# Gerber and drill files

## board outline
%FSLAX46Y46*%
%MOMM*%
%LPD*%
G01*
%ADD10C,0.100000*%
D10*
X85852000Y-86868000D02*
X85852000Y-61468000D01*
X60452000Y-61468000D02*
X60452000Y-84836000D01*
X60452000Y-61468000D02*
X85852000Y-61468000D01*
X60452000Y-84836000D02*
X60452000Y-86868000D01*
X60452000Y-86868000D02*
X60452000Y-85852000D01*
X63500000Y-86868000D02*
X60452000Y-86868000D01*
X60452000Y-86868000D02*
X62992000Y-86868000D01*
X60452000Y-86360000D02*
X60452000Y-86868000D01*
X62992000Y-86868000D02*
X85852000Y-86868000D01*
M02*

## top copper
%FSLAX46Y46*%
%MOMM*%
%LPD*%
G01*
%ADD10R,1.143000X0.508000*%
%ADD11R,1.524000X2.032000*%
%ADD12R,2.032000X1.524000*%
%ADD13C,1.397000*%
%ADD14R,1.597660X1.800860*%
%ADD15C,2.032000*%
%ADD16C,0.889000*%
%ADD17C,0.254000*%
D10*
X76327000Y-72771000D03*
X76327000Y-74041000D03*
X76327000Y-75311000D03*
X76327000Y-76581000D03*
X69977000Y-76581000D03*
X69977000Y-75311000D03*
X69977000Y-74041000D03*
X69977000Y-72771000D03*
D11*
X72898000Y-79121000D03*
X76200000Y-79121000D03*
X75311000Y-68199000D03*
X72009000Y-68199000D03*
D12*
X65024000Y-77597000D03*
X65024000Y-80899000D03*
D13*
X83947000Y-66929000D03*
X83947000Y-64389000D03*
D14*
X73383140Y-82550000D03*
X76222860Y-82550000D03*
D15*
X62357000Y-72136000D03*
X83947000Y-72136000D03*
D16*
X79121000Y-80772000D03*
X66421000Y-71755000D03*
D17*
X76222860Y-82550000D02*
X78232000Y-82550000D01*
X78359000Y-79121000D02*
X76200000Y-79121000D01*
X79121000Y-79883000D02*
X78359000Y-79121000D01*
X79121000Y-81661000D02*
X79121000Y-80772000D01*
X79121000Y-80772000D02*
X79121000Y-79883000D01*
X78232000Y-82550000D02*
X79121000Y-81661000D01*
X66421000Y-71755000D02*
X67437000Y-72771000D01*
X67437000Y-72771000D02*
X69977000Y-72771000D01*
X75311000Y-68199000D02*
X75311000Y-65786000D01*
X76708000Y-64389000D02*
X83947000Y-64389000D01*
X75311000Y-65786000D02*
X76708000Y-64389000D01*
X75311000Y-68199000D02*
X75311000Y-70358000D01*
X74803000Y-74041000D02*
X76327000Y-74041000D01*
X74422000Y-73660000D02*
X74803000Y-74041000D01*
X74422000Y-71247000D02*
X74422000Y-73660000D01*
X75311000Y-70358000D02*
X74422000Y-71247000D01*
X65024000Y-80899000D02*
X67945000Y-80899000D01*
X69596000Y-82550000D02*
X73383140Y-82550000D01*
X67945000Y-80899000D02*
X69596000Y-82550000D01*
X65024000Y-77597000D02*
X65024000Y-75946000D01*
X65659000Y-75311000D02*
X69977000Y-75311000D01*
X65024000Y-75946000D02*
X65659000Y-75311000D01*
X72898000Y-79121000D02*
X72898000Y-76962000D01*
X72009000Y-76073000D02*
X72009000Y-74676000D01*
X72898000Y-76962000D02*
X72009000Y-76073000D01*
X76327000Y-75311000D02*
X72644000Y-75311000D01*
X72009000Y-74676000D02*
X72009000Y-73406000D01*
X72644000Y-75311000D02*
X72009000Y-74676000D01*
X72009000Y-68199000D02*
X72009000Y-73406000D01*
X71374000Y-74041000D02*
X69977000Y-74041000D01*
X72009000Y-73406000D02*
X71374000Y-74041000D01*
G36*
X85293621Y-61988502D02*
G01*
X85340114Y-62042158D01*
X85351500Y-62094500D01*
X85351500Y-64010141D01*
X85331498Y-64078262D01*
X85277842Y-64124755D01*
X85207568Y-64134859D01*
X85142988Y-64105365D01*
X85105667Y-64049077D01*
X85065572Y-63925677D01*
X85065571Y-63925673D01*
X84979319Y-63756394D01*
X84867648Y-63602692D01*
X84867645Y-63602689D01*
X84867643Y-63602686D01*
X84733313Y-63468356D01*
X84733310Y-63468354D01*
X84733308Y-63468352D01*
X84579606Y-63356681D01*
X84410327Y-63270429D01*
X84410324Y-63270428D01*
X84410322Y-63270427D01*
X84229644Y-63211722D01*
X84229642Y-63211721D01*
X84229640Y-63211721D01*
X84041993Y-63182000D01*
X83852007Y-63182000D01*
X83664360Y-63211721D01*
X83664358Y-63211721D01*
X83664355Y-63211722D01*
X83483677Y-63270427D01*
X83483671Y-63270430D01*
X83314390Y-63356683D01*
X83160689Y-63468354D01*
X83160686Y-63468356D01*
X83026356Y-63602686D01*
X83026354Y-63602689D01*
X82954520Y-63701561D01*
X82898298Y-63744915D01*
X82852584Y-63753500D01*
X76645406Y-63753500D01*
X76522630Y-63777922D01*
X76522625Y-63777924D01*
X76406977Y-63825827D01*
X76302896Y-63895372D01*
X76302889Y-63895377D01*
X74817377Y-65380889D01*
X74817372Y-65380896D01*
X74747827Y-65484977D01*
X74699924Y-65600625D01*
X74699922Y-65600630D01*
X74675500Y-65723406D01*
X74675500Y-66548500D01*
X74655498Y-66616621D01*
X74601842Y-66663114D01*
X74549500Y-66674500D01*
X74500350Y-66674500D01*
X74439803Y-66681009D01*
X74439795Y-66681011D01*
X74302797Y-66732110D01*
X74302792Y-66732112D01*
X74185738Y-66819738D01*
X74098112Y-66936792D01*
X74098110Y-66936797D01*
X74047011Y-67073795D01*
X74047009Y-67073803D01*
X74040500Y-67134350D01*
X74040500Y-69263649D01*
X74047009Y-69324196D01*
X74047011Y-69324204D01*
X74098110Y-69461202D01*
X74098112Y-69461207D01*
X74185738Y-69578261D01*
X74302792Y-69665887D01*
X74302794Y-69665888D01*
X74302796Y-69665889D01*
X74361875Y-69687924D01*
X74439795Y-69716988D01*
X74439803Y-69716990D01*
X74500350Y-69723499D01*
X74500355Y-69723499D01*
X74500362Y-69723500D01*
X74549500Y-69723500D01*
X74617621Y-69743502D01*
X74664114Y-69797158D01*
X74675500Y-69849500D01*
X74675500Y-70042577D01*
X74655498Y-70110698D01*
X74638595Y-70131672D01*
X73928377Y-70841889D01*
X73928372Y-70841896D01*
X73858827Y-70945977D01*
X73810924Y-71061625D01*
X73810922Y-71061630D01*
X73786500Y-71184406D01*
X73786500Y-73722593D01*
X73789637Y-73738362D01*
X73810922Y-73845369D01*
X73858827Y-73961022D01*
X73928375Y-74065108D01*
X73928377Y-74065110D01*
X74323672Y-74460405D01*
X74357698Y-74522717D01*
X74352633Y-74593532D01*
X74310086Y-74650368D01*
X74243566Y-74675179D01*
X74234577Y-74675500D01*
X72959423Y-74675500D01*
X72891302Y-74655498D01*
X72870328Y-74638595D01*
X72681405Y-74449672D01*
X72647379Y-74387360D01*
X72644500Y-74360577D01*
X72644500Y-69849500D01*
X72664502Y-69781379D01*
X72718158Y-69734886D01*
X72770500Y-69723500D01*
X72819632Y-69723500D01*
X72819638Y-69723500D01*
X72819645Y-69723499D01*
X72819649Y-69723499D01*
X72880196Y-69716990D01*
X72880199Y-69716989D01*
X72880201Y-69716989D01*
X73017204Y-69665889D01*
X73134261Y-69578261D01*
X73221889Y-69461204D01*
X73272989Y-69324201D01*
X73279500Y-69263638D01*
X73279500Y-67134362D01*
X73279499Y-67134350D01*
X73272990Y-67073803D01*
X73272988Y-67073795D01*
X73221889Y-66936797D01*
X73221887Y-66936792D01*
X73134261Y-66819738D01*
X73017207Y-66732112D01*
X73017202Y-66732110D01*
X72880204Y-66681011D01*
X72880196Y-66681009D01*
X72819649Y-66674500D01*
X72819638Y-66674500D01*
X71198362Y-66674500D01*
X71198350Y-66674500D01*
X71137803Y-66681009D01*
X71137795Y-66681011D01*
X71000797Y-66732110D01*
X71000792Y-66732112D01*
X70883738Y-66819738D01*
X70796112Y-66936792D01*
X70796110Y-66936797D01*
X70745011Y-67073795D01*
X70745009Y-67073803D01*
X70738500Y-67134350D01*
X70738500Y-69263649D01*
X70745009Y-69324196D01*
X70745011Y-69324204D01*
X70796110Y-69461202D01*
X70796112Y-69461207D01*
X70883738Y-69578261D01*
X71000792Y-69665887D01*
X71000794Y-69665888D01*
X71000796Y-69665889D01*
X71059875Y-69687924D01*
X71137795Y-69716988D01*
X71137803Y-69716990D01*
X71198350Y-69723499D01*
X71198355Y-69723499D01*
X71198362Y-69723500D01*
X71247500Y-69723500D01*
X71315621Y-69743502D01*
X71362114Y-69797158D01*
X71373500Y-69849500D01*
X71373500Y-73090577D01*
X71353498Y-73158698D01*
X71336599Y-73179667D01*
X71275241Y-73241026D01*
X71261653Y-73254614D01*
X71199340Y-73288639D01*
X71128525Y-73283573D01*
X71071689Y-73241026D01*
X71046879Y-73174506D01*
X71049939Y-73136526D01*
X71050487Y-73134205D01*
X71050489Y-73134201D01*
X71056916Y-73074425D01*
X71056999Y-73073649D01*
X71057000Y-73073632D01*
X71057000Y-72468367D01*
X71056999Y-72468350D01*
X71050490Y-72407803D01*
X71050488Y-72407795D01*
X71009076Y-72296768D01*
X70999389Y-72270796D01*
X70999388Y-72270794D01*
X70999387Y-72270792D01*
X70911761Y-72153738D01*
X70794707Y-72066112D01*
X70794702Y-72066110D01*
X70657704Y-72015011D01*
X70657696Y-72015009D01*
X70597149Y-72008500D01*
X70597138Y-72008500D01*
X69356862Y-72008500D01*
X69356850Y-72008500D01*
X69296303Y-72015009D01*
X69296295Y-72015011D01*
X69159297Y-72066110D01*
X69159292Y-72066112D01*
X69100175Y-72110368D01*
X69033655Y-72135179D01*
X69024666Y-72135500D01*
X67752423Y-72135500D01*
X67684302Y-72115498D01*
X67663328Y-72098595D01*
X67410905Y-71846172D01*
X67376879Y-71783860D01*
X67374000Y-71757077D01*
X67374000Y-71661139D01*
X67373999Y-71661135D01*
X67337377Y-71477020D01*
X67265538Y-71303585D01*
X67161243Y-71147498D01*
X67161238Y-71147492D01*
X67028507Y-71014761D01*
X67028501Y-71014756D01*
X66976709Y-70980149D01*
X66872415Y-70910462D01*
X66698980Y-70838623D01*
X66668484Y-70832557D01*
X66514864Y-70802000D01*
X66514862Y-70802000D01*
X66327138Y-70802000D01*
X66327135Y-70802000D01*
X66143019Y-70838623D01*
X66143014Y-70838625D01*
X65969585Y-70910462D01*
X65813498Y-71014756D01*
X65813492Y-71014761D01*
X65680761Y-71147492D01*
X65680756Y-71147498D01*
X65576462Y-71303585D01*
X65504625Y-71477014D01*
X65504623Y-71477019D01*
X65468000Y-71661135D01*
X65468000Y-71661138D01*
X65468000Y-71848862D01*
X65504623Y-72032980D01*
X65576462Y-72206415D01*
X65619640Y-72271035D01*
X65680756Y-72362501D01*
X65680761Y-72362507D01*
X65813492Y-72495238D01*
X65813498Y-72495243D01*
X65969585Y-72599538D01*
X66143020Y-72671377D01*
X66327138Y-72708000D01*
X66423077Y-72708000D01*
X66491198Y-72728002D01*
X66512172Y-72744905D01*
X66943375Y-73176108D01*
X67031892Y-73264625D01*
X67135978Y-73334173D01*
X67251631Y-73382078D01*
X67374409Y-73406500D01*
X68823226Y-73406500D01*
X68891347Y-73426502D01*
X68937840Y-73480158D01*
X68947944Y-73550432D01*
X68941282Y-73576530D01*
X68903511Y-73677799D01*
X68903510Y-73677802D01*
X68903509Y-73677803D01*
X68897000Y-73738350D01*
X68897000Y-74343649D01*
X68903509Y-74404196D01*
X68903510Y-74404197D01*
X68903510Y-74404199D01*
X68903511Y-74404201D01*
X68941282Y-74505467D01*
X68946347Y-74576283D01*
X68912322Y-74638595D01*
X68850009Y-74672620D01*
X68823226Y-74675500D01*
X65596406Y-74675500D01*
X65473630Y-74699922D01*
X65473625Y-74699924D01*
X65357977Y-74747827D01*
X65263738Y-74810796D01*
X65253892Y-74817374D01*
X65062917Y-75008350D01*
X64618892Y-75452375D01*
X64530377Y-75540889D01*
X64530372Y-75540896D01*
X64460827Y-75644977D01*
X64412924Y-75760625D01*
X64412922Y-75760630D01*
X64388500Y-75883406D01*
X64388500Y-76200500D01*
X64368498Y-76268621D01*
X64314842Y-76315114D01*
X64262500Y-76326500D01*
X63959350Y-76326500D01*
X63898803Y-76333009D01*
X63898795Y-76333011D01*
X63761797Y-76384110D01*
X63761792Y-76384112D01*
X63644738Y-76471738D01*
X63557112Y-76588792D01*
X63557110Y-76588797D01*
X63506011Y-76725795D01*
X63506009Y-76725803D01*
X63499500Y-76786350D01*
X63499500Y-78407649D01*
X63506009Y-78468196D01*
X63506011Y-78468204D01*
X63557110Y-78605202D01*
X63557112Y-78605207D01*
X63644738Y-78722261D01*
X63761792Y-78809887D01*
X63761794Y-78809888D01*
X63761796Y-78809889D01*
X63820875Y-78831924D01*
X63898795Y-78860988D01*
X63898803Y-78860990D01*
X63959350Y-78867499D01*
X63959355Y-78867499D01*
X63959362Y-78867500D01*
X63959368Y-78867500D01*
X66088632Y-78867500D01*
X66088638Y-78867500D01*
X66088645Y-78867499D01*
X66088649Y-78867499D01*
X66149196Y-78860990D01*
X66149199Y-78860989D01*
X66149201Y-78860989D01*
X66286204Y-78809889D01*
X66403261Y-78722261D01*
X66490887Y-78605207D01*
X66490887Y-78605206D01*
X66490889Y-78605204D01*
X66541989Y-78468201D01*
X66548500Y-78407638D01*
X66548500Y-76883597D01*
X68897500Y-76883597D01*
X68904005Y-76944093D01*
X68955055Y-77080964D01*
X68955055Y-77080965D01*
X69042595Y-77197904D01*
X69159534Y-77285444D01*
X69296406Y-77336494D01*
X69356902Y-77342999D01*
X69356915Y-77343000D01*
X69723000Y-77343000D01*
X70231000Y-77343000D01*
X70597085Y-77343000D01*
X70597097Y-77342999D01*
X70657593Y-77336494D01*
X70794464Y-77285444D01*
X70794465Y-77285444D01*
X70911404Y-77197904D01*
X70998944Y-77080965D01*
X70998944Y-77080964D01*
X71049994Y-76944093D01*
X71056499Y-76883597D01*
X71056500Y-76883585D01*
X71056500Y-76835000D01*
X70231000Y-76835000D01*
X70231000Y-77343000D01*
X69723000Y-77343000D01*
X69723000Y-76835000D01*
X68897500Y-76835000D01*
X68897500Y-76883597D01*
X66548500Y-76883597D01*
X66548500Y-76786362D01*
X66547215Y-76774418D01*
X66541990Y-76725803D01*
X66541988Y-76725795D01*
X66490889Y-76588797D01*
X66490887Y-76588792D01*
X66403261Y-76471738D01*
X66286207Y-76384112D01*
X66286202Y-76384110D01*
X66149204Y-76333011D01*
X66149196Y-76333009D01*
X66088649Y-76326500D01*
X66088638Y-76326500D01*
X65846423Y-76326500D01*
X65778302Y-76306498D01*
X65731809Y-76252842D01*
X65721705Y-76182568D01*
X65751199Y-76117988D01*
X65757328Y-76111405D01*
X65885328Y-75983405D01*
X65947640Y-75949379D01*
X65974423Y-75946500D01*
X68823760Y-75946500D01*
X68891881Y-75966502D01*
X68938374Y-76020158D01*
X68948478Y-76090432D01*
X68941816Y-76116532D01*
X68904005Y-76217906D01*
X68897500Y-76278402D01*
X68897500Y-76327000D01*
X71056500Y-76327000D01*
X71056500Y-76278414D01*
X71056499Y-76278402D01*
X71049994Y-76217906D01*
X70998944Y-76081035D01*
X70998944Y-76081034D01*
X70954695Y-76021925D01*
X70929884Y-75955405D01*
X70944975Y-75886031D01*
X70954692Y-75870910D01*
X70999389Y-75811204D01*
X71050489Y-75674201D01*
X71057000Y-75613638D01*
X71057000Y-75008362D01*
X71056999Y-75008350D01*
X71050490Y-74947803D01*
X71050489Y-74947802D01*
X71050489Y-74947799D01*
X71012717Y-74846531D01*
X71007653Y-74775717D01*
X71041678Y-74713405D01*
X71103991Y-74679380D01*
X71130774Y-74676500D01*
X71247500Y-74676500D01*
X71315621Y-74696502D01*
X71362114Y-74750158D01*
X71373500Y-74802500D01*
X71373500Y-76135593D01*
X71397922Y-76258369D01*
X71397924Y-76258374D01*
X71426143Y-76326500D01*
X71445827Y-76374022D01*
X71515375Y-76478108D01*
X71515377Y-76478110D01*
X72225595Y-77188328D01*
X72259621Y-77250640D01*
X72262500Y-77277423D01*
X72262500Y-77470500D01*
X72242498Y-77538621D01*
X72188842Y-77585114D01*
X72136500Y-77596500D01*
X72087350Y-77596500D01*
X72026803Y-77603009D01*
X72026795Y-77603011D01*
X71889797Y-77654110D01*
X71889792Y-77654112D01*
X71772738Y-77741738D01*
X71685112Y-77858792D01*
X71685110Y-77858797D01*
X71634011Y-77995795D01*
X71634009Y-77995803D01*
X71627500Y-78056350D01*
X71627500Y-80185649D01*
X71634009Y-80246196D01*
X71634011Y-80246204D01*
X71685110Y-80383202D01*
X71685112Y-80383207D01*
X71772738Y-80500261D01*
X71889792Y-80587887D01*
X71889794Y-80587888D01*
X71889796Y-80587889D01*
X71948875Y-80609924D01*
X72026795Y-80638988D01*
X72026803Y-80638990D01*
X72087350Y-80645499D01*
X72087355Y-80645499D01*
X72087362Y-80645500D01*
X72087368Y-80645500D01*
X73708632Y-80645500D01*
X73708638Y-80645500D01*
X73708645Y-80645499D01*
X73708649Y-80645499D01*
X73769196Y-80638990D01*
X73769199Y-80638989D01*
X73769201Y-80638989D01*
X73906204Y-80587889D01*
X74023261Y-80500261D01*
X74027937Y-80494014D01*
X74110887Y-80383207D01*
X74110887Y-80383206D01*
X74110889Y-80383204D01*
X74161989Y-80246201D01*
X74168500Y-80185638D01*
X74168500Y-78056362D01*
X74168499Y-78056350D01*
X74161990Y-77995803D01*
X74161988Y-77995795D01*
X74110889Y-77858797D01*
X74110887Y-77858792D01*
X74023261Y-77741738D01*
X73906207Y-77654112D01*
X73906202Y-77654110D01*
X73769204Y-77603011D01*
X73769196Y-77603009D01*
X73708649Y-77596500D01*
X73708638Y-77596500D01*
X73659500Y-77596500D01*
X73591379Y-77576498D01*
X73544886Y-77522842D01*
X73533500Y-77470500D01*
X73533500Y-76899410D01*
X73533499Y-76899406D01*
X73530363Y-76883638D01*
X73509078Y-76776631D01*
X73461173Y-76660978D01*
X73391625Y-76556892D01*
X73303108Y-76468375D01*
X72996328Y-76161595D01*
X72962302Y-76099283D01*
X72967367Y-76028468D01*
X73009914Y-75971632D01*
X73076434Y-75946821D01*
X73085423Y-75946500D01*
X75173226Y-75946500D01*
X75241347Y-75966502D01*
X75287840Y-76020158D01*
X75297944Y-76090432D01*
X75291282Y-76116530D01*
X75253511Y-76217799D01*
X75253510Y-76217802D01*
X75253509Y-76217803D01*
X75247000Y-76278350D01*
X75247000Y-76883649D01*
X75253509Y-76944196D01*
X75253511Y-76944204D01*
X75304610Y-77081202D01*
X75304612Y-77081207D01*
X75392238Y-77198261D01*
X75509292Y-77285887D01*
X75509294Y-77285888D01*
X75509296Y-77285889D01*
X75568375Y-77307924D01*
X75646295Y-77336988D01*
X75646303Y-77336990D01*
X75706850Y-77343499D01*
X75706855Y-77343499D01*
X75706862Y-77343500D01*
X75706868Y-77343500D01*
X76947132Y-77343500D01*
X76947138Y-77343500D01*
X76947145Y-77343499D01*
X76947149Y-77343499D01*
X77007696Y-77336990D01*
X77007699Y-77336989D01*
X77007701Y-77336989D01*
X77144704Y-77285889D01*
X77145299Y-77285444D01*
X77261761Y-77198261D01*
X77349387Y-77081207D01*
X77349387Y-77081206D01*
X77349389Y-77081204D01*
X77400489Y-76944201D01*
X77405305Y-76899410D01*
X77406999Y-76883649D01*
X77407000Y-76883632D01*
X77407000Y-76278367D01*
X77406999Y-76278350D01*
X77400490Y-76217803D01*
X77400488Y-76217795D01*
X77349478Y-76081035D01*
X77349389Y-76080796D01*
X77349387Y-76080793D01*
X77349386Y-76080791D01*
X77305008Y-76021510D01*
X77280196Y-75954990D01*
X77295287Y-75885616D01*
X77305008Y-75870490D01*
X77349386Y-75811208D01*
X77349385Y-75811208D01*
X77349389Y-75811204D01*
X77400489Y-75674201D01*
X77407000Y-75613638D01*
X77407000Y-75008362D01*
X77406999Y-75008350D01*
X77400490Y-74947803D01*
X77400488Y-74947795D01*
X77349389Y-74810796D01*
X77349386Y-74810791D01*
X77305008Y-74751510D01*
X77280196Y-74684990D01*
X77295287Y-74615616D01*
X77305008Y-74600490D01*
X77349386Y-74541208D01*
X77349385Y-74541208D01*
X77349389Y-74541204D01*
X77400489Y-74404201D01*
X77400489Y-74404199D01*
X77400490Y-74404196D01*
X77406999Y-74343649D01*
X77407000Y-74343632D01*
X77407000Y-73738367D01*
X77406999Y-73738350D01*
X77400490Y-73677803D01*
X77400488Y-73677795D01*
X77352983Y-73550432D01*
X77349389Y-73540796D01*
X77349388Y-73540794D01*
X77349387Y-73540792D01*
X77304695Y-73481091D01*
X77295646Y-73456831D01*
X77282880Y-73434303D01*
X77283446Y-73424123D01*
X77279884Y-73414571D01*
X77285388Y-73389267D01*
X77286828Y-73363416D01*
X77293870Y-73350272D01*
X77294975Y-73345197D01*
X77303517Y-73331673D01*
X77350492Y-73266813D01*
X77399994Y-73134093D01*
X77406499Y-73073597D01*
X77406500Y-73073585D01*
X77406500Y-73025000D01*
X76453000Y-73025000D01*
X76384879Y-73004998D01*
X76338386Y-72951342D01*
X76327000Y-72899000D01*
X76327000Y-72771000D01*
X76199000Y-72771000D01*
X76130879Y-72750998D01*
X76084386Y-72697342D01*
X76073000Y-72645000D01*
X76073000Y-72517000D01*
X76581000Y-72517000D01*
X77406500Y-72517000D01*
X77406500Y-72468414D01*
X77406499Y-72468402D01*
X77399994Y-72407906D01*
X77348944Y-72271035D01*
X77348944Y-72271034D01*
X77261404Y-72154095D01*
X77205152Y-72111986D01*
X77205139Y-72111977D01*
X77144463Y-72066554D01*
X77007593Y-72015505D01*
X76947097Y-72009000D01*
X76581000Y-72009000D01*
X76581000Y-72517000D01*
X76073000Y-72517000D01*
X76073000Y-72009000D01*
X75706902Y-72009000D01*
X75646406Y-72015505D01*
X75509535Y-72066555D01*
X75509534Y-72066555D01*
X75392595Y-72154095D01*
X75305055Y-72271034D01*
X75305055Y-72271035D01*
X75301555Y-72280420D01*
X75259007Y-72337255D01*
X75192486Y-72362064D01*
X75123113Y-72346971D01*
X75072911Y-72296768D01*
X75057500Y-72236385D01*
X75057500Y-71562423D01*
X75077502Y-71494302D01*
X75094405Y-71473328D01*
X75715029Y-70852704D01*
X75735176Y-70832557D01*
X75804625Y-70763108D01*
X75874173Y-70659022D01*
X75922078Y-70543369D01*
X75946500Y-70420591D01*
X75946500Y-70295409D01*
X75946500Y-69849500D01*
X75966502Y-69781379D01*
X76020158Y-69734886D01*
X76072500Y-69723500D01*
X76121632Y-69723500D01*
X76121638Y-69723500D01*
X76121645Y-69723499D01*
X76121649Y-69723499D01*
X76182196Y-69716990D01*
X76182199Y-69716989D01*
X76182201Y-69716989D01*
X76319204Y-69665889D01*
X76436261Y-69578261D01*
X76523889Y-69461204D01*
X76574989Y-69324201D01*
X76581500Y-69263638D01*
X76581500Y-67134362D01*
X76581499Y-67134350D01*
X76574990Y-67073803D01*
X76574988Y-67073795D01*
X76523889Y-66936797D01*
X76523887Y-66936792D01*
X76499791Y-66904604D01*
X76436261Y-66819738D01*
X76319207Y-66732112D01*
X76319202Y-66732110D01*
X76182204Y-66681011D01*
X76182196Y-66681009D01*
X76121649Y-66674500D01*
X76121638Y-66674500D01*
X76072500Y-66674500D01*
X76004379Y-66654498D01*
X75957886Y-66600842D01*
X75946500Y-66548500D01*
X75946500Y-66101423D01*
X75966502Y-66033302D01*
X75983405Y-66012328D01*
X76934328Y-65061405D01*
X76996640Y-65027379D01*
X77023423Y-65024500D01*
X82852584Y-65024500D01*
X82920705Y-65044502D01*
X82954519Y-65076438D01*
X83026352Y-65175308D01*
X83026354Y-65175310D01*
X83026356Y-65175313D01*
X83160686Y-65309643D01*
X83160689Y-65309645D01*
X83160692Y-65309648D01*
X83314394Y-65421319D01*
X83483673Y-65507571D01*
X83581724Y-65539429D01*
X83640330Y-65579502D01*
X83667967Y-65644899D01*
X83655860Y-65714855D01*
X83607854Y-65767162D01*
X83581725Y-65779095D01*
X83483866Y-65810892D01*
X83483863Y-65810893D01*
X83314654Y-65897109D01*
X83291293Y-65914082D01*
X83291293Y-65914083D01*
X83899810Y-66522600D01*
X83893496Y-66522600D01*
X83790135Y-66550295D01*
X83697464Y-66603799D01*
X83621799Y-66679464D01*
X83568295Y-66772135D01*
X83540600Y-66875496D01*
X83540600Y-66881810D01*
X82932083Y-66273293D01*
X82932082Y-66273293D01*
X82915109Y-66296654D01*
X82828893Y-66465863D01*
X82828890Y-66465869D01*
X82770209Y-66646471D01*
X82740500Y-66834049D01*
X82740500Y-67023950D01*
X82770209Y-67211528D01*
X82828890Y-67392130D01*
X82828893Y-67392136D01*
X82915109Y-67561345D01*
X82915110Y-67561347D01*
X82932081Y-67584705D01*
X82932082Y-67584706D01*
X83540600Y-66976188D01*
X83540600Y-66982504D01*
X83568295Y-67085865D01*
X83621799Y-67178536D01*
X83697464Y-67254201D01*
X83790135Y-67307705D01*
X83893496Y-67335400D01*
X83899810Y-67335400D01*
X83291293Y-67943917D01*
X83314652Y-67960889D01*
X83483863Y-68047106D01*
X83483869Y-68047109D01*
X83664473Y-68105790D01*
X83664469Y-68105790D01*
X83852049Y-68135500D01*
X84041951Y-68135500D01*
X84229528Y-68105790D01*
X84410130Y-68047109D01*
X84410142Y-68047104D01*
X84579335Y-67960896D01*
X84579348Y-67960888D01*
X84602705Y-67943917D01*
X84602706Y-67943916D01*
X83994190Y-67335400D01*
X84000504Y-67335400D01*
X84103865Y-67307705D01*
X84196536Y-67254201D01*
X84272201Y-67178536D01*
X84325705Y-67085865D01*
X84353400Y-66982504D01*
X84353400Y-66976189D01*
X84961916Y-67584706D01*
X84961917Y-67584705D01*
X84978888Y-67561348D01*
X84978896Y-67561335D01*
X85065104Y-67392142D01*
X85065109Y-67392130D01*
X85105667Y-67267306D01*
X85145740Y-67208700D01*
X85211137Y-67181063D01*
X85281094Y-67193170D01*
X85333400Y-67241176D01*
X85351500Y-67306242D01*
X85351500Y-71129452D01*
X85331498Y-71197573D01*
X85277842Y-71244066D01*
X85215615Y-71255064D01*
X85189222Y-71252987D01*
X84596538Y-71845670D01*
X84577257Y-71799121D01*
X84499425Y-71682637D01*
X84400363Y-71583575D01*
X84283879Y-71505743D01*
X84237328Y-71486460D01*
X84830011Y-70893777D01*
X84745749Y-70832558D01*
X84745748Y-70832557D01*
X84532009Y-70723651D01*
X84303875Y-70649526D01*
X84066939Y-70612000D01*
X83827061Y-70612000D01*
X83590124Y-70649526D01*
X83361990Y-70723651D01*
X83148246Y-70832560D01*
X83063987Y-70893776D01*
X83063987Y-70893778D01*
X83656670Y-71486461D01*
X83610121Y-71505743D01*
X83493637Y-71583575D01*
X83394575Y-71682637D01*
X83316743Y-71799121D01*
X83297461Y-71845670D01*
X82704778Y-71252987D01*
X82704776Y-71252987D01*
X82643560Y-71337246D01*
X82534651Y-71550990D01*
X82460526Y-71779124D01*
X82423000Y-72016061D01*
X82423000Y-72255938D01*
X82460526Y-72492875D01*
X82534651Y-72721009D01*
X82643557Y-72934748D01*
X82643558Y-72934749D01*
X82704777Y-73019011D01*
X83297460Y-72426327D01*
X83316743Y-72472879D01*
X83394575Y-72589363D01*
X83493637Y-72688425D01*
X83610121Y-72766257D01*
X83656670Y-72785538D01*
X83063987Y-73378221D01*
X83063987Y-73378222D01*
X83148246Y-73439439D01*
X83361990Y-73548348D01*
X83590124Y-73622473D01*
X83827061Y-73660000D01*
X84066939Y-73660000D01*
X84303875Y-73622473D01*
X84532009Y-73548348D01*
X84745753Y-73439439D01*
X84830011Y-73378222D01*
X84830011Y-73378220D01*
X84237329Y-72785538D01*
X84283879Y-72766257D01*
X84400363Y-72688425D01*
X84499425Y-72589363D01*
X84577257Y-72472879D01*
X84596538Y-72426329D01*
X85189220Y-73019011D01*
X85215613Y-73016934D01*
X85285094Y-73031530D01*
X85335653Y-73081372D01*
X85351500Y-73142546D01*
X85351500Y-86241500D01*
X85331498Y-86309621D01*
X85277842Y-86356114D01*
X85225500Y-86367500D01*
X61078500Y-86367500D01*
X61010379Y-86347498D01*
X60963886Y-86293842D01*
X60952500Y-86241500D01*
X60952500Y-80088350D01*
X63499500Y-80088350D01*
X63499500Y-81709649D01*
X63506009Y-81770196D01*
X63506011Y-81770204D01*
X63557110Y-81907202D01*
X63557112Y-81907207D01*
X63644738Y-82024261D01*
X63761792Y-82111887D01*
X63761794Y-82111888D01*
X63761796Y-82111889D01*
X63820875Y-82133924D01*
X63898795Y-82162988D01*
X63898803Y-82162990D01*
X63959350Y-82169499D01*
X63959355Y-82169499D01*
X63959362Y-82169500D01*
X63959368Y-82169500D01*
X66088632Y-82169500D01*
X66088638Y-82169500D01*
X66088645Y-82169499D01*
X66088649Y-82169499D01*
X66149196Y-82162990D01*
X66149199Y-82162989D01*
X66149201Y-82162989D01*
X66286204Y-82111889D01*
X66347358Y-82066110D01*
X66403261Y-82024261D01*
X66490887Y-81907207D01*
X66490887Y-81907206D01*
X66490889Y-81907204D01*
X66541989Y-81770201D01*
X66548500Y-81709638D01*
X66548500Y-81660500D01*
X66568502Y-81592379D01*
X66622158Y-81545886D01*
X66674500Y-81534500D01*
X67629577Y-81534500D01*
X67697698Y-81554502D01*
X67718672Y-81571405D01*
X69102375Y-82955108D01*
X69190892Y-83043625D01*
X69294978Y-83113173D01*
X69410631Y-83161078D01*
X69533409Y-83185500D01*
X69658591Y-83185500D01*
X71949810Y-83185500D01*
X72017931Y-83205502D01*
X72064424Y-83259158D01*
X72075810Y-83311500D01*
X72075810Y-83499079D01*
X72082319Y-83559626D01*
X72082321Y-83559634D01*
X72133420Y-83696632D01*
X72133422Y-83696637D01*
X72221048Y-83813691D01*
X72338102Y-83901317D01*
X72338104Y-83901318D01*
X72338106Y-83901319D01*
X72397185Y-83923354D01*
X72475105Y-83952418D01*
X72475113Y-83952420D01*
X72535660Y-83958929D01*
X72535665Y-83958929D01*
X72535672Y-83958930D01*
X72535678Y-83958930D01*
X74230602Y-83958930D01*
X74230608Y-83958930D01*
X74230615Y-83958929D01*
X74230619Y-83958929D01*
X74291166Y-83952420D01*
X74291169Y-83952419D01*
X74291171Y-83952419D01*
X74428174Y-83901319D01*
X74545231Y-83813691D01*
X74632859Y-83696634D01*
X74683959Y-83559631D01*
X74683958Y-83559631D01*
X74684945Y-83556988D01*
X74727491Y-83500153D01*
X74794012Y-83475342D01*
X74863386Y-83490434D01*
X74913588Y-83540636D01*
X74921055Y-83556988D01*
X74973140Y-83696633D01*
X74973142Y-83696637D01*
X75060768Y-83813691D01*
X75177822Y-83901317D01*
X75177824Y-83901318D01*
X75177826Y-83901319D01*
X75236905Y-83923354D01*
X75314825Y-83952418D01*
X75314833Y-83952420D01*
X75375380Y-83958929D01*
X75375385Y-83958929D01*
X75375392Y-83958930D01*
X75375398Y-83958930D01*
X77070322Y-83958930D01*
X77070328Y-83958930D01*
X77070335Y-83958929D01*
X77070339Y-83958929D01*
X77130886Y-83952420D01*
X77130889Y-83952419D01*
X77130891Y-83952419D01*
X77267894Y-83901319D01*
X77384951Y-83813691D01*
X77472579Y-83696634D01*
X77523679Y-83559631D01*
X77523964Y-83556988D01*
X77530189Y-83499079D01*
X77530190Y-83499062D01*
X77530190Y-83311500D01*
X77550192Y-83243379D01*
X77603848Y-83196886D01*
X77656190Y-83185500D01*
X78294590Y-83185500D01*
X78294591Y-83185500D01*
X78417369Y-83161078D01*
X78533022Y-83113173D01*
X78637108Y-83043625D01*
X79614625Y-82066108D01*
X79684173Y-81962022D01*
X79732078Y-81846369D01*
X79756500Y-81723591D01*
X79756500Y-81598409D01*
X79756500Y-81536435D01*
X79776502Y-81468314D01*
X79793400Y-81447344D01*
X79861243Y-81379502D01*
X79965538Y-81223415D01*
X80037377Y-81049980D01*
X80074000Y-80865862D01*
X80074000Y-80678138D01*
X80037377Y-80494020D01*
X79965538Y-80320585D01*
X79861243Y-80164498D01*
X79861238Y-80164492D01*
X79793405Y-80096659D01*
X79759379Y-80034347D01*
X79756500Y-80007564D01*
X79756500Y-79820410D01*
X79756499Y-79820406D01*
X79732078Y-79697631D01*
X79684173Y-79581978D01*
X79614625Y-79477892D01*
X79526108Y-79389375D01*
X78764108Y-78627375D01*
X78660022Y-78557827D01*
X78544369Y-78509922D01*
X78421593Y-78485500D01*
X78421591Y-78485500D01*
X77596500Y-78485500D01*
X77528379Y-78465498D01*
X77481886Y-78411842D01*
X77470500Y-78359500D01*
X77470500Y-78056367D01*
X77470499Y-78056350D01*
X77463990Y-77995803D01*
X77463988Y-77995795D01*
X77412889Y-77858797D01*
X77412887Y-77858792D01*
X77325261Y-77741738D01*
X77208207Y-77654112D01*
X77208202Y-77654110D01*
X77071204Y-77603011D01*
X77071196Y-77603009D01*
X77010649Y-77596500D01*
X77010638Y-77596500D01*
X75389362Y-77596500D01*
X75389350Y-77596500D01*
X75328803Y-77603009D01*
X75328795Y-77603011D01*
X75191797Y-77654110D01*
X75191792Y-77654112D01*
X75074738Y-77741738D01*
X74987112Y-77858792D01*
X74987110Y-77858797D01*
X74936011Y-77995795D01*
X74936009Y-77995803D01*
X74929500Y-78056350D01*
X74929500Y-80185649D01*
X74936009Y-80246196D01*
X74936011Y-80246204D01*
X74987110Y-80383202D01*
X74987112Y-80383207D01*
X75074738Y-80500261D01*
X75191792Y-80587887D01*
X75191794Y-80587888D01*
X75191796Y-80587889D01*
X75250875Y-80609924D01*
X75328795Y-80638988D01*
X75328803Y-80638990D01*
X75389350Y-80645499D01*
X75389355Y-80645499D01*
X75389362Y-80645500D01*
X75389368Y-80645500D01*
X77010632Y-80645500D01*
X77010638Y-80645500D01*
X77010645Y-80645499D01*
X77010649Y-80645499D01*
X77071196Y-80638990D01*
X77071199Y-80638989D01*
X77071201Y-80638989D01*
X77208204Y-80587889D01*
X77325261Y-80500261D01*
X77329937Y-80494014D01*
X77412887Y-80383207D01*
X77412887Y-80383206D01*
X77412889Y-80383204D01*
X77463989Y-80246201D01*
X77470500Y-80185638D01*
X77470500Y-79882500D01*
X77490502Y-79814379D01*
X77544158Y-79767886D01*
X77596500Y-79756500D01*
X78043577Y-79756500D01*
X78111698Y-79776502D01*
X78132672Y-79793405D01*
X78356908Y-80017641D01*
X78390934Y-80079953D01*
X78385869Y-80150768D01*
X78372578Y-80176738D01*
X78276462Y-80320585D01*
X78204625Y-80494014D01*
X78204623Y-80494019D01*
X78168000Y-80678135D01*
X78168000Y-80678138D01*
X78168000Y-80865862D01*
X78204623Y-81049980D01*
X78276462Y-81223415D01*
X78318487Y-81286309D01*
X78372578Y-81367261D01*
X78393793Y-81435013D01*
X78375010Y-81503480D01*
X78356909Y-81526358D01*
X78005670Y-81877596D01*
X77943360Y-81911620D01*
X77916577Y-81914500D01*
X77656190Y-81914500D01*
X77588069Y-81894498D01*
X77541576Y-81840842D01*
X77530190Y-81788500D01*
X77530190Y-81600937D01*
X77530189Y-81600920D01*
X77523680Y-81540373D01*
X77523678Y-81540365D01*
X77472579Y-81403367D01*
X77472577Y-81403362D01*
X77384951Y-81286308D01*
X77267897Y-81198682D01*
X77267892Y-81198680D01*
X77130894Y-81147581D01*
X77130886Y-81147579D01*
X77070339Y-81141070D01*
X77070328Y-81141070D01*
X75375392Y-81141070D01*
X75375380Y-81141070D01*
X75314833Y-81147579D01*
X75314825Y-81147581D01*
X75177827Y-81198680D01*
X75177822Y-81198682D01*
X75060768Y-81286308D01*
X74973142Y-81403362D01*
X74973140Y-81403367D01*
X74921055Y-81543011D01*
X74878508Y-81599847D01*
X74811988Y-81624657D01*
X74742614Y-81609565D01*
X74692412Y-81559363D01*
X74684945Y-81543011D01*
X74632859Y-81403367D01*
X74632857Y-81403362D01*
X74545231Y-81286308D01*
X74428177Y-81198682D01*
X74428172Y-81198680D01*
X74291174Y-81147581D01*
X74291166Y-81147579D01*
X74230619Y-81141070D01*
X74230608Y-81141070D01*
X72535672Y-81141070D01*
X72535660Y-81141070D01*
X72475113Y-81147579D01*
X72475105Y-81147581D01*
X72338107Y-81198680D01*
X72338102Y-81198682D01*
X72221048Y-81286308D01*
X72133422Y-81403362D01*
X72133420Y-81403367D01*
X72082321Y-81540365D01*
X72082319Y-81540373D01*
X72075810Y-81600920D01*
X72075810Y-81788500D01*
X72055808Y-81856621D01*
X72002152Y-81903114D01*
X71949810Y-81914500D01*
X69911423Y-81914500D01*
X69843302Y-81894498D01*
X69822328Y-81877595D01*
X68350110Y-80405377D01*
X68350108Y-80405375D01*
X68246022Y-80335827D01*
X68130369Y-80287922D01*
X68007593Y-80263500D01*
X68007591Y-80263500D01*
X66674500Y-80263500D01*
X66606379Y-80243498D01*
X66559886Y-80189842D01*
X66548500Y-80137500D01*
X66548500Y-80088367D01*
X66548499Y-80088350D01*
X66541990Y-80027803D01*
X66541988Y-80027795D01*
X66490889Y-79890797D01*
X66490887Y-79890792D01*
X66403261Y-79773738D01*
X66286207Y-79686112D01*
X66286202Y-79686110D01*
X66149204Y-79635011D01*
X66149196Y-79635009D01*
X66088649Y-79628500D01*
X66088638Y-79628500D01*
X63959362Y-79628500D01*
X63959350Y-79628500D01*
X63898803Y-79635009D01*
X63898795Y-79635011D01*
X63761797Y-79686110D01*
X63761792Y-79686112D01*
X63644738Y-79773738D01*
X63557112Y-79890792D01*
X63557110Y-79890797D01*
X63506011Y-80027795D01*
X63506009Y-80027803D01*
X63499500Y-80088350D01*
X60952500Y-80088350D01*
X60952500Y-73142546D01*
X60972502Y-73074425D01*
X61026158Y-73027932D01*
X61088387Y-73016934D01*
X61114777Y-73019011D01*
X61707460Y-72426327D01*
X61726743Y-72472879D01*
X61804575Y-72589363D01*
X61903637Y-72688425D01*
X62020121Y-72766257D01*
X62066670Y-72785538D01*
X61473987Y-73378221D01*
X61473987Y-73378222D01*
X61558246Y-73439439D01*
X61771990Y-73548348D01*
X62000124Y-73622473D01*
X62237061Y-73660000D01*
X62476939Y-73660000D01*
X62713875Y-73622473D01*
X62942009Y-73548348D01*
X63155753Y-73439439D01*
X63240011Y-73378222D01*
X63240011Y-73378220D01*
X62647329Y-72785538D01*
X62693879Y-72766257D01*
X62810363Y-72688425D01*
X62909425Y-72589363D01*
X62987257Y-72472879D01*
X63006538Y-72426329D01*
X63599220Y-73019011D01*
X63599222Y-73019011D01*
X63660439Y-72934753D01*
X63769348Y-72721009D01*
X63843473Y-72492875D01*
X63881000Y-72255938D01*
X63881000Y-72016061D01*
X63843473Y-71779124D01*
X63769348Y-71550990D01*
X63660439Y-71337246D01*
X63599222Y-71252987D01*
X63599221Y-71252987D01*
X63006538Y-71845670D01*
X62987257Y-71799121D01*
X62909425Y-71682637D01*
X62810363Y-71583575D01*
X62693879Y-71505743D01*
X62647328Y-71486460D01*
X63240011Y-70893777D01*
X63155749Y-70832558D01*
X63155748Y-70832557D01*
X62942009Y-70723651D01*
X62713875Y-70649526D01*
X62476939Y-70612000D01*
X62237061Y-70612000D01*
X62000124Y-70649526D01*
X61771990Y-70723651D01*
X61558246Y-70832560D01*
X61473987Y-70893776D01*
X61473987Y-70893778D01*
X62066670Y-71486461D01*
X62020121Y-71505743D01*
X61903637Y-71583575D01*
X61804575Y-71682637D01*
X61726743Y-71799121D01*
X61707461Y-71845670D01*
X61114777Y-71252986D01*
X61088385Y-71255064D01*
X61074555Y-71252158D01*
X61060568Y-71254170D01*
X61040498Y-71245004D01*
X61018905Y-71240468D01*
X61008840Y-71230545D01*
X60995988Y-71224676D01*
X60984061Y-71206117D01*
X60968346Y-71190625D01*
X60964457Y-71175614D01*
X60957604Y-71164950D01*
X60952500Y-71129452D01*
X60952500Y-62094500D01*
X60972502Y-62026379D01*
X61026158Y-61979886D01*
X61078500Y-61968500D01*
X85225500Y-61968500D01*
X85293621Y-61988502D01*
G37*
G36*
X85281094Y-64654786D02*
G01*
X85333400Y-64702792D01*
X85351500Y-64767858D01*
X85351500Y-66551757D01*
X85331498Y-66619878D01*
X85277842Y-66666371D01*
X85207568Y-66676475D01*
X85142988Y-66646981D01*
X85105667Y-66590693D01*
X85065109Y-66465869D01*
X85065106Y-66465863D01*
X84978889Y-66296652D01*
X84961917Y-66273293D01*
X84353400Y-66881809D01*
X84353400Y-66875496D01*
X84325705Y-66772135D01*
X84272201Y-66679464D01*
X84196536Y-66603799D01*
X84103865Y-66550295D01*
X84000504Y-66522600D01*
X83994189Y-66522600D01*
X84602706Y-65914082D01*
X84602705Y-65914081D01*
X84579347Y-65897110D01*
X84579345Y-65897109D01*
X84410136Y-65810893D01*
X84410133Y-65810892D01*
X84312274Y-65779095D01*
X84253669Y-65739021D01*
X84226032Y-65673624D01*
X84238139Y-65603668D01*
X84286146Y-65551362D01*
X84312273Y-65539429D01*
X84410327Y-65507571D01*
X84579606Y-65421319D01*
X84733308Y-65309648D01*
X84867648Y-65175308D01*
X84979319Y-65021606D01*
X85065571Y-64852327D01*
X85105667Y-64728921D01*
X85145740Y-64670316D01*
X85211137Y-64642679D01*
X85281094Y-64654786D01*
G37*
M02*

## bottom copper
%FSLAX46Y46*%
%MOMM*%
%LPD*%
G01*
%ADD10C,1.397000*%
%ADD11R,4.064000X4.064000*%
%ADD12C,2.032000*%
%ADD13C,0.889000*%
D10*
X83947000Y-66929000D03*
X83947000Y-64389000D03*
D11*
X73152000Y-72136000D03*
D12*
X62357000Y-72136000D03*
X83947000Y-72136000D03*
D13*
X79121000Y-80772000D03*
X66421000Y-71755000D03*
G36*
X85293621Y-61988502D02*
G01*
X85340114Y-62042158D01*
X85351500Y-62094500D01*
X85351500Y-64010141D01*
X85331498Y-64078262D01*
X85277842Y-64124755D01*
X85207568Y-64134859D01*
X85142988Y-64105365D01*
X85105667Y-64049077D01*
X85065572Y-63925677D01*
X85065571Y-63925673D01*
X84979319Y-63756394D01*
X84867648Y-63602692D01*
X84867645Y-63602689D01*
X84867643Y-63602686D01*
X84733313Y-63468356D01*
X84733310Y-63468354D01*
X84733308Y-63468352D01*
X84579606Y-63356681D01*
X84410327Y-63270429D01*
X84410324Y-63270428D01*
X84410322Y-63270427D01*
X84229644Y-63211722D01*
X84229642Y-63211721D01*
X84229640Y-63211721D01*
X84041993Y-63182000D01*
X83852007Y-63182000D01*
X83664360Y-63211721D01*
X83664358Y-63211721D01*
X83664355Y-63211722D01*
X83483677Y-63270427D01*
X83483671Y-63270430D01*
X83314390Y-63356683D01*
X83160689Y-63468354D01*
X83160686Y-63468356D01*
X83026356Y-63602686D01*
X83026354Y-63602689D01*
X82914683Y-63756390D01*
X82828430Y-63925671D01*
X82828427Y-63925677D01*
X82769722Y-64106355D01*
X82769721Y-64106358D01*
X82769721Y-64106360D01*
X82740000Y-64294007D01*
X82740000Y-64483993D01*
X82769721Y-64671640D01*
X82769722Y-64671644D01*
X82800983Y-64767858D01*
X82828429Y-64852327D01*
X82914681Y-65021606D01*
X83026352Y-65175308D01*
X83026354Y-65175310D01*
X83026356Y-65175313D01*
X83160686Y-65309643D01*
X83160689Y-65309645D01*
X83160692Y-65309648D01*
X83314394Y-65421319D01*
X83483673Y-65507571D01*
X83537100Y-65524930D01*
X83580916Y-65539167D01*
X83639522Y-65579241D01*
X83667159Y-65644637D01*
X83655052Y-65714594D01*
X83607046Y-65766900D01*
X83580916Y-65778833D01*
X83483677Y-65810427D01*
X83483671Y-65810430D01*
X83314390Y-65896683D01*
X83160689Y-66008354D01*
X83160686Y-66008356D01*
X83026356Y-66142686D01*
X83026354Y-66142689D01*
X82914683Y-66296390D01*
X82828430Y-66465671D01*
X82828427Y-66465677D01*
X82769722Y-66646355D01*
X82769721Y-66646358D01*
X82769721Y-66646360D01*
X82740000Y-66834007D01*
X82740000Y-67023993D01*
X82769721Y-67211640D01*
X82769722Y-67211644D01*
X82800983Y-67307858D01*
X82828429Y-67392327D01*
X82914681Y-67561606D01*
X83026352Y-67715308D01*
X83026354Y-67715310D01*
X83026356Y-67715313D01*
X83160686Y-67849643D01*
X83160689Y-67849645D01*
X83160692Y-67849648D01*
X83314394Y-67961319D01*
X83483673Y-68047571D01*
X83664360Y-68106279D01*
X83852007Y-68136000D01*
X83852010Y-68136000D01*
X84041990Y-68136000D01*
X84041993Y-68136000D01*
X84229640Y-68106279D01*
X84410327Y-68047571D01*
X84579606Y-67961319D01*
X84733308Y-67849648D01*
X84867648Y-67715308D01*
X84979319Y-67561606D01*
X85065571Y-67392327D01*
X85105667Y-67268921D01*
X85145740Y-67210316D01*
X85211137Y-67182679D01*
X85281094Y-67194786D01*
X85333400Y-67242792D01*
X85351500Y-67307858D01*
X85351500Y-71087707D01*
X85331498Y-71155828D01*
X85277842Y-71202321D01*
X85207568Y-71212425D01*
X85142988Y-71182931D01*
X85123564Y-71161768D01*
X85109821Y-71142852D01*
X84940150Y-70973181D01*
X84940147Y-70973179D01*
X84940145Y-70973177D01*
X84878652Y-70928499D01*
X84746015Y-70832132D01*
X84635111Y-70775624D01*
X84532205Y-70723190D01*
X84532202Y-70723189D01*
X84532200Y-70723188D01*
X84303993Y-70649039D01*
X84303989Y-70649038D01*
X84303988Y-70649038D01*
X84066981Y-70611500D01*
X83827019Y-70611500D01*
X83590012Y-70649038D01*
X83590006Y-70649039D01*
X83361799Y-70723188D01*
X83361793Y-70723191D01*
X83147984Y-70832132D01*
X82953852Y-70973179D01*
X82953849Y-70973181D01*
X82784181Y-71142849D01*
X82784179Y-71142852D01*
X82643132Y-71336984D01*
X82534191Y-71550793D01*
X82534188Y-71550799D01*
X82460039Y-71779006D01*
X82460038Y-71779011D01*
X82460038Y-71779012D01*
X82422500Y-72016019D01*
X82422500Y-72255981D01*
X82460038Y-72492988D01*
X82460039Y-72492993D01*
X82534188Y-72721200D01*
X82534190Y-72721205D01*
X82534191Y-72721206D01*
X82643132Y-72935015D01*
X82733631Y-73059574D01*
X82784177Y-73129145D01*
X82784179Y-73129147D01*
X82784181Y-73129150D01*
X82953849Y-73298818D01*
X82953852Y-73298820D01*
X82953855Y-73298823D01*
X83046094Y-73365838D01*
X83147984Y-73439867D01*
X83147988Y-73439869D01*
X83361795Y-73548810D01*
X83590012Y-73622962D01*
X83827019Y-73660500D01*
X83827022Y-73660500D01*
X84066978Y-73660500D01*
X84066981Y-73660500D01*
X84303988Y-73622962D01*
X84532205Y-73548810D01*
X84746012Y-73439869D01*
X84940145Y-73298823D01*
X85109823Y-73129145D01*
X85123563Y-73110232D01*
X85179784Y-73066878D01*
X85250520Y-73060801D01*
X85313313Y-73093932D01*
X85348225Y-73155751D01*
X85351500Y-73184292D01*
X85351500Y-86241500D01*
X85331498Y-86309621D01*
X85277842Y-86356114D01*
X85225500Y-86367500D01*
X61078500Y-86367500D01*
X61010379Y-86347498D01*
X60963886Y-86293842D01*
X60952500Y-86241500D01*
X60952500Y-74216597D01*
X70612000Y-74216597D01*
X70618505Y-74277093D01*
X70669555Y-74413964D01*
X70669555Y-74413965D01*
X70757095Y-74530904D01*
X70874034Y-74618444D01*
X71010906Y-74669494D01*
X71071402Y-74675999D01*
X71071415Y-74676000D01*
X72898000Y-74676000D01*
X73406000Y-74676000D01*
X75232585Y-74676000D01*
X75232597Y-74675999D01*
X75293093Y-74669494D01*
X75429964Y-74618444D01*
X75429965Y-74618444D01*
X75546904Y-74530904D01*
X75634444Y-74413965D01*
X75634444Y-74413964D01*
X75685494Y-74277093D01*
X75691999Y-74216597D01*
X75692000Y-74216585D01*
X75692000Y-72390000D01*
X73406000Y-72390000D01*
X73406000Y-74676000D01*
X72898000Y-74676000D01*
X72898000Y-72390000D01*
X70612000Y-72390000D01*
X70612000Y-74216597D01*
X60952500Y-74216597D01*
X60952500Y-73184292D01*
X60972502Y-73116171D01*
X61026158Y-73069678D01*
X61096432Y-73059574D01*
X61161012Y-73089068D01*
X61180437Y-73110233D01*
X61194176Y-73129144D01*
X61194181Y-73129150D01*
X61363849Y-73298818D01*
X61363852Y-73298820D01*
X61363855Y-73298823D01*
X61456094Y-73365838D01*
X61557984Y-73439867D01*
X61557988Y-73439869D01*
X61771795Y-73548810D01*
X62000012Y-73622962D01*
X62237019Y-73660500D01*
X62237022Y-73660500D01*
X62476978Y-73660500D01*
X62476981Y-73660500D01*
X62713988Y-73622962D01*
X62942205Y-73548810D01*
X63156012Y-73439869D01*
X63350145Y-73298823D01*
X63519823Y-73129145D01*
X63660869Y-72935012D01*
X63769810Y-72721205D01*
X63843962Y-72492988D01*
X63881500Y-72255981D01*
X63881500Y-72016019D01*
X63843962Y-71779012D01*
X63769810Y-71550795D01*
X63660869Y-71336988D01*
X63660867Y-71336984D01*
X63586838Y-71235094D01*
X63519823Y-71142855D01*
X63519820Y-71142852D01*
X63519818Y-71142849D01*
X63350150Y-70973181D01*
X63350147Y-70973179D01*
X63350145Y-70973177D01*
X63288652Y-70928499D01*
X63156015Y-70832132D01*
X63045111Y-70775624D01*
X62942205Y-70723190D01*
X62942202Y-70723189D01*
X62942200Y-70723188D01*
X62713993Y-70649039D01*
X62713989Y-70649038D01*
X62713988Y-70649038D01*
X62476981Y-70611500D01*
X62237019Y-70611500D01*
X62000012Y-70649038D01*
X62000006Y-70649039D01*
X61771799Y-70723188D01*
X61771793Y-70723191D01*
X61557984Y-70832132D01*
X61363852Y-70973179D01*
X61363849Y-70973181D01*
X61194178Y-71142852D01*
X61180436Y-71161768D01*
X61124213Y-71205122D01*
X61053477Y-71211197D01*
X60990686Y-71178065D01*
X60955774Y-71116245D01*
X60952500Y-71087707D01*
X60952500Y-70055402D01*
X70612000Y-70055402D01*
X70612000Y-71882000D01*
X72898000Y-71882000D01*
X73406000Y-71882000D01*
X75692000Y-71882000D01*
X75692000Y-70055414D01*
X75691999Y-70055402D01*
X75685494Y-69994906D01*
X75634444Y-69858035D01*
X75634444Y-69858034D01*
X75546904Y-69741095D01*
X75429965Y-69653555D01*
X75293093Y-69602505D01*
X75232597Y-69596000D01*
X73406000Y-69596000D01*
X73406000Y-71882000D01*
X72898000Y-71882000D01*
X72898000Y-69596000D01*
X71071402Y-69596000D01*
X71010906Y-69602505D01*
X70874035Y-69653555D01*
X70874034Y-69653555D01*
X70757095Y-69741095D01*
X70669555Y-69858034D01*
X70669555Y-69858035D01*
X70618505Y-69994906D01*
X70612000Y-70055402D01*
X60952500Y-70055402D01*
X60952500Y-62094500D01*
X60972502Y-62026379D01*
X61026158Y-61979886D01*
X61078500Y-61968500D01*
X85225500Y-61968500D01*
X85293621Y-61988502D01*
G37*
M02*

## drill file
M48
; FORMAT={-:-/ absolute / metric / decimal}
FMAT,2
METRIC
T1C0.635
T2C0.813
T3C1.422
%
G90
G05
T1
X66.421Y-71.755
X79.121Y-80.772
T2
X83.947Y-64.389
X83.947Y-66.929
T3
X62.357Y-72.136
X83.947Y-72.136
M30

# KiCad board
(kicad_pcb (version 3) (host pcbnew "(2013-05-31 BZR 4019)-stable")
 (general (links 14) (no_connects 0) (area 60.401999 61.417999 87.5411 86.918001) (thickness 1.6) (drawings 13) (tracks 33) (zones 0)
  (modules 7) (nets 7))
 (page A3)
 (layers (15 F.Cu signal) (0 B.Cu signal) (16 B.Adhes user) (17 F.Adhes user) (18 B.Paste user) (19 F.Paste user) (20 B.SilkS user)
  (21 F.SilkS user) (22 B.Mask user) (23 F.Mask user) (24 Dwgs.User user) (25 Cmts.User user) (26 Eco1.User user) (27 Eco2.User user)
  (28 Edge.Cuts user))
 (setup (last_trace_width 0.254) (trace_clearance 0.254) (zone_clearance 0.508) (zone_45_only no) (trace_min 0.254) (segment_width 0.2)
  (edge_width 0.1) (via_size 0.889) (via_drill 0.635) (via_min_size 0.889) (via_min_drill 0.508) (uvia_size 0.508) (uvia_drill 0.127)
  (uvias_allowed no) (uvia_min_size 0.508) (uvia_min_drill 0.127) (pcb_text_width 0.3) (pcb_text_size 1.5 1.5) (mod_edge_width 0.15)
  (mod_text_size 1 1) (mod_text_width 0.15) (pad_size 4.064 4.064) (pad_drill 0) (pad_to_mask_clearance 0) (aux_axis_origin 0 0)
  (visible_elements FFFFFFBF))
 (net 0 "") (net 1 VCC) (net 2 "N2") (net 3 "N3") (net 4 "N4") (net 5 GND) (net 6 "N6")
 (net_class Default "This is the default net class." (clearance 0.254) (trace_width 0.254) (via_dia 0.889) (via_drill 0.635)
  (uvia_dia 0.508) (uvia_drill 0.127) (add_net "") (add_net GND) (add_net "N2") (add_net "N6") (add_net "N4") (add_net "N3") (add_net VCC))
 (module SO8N (layer F.Cu) (at 73.152 74.676 270)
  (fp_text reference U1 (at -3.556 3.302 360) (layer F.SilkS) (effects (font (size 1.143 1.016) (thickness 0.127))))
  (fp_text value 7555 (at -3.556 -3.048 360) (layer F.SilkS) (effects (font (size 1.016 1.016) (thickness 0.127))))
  (pad 8 smd rect (at -1.905 -3.175 270) (size 0.508 1.143) (layers F.Cu F.Paste F.Mask) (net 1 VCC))
  (pad 7 smd rect (at -0.635 -3.175 270) (size 0.508 1.143) (layers F.Cu F.Paste F.Mask) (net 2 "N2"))
  (pad 6 smd rect (at 0.635 -3.175 270) (size 0.508 1.143) (layers F.Cu F.Paste F.Mask) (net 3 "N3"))
  (pad 5 smd rect (at 1.905 -3.175 270) (size 0.508 1.143) (layers F.Cu F.Paste F.Mask))
  (pad 4 smd rect (at 1.905 3.175 270) (size 0.508 1.143) (layers F.Cu F.Paste F.Mask) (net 1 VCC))
  (pad 3 smd rect (at 0.635 3.175 270) (size 0.508 1.143) (layers F.Cu F.Paste F.Mask) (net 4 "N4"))
  (pad 2 smd rect (at -0.635 3.175 270) (size 0.508 1.143) (layers F.Cu F.Paste F.Mask) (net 3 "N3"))
  (pad 1 smd rect (at -1.905 3.175 270) (size 0.508 1.143) (layers F.Cu F.Paste F.Mask) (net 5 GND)))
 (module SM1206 (layer F.Cu) (at 74.549 79.121)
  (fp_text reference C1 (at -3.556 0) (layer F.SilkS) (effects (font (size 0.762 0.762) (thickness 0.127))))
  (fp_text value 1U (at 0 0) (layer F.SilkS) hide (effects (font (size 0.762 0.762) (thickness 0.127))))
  (pad 1 smd rect (at -1.651 0) (size 1.524 2.032) (layers F.Cu F.Paste F.Mask) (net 3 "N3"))
  (pad 2 smd rect (at 1.651 0) (size 1.524 2.032) (layers F.Cu F.Paste F.Mask) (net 5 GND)))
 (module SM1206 (layer F.Cu) (at 73.66 68.199 180)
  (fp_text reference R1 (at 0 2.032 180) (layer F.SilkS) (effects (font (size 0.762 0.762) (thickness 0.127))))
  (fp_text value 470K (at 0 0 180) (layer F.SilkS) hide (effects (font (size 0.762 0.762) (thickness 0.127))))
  (pad 1 smd rect (at -1.651 0 180) (size 1.524 2.032) (layers F.Cu F.Paste F.Mask) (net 2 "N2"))
  (pad 2 smd rect (at 1.651 0 180) (size 1.524 2.032) (layers F.Cu F.Paste F.Mask) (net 3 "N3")))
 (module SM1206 (layer F.Cu) (at 65.024 79.248 270)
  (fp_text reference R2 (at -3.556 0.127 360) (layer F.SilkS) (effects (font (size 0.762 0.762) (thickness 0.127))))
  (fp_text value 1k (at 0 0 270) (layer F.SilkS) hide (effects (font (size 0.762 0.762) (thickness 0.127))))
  (pad 1 smd rect (at -1.651 0 270) (size 1.524 2.032) (layers F.Cu F.Paste F.Mask) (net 4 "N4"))
  (pad 2 smd rect (at 1.651 0 270) (size 1.524 2.032) (layers F.Cu F.Paste F.Mask) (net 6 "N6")))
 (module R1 (layer F.Cu) (at 83.947 65.659 90) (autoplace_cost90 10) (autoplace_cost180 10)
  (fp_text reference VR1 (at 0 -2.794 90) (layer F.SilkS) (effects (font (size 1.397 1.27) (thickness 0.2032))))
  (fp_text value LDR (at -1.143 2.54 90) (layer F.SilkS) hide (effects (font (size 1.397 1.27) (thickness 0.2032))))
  (pad 1 thru_hole circle (at -1.27 0 90) (size 1.397 1.397) (drill 0.8128) (layers *.Cu *.Mask F.SilkS) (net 1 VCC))
  (pad 2 thru_hole circle (at 1.27 0 90) (size 1.397 1.397) (drill 0.8128) (layers *.Cu *.Mask F.SilkS) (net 2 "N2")))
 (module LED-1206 (layer F.Cu) (at 74.803 82.55)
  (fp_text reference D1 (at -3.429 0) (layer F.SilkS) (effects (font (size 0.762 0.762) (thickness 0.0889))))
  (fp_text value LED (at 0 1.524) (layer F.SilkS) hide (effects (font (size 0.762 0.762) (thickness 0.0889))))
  (pad 1 smd rect (at -1.41986 0) (size 1.59766 1.80086) (layers F.Cu F.Paste F.Mask) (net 6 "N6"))
  (pad 2 smd rect (at 1.41986 0) (size 1.59766 1.80086) (layers F.Cu F.Paste F.Mask) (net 5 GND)))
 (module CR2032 (layer B.Cu) (at 73.152 72.136 180)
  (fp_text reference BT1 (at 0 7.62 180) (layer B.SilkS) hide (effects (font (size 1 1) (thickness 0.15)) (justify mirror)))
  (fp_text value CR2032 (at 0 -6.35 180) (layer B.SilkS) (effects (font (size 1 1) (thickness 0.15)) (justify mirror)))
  (pad 2 smd rect (at 0 0 180) (size 4.064 4.064) (layers B.Cu B.Paste B.Mask) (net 5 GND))
  (pad 1 thru_hole circle (at 10.795 0 180) (size 2.032 2.032) (drill 1.4224) (layers *.Cu *.Mask B.SilkS) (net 1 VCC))
  (pad 1 thru_hole circle (at -10.795 0 180) (size 2.032 2.032) (drill 1.4224) (layers *.Cu *.Mask B.SilkS) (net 1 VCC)))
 (gr_line (start 85.852 86.868) (end 85.852 61.468) (angle 90) (layer Edge.Cuts) (width 0.1))
 (gr_line (start 60.452 61.468) (end 60.452 84.836) (angle 90) (layer Edge.Cuts) (width 0.1))
 (gr_line (start 60.452 61.468) (end 85.852 61.468) (angle 90) (layer Edge.Cuts) (width 0.1))
 (gr_line (start 60.452 84.836) (end 60.452 86.868) (angle 90) (layer Edge.Cuts) (width 0.1))
 (gr_line (start 60.452 86.868) (end 60.452 85.852) (angle 90) (layer Edge.Cuts) (width 0.1))
 (gr_line (start 63.5 86.868) (end 60.452 86.868) (angle 90) (layer Edge.Cuts) (width 0.1))
 (gr_line (start 60.452 86.868) (end 62.992 86.868) (angle 90) (layer Edge.Cuts) (width 0.1))
 (gr_line (start 60.452 86.36) (end 60.452 86.868) (angle 90) (layer Edge.Cuts) (width 0.1))
 (gr_line (start 62.992 86.868) (end 85.852 86.868) (angle 90) (layer Edge.Cuts) (width 0.1))
 (via (at 79.121 80.772) (size 0.889) (layers F.Cu B.Cu) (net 5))
 (segment (start 76.22286 82.55) (end 78.232 82.55) (width 0.254) (layer F.Cu) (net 5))
 (segment (start 78.359 79.121) (end 76.2 79.121) (width 0.254) (layer F.Cu) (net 5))
 (segment (start 79.121 79.883) (end 78.359 79.121) (width 0.254) (layer F.Cu) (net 5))
 (segment (start 79.121 81.661) (end 79.121 80.772) (width 0.254) (layer F.Cu) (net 5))
 (segment (start 79.121 80.772) (end 79.121 79.883) (width 0.254) (layer F.Cu) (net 5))
 (segment (start 78.232 82.55) (end 79.121 81.661) (width 0.254) (layer F.Cu) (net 5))
 (via (at 66.421 71.755) (size 0.889) (layers F.Cu B.Cu) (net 5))
 (segment (start 66.421 71.755) (end 67.437 72.771) (width 0.254) (layer F.Cu) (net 5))
 (segment (start 67.437 72.771) (end 69.977 72.771) (width 0.254) (layer F.Cu) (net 5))
 (segment (start 75.311 68.199) (end 75.311 65.786) (width 0.254) (layer F.Cu) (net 2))
 (segment (start 76.708 64.389) (end 83.947 64.389) (width 0.254) (layer F.Cu) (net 2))
 (segment (start 75.311 65.786) (end 76.708 64.389) (width 0.254) (layer F.Cu) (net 2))
 (segment (start 75.311 68.199) (end 75.311 70.358) (width 0.254) (layer F.Cu) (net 2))
 (segment (start 74.803 74.041) (end 76.327 74.041) (width 0.254) (layer F.Cu) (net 2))
 (segment (start 74.422 73.66) (end 74.803 74.041) (width 0.254) (layer F.Cu) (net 2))
 (segment (start 74.422 71.247) (end 74.422 73.66) (width 0.254) (layer F.Cu) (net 2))
 (segment (start 75.311 70.358) (end 74.422 71.247) (width 0.254) (layer F.Cu) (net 2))
 (segment (start 65.024 80.899) (end 67.945 80.899) (width 0.254) (layer F.Cu) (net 6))
 (segment (start 69.596 82.55) (end 73.38314 82.55) (width 0.254) (layer F.Cu) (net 6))
 (segment (start 67.945 80.899) (end 69.596 82.55) (width 0.254) (layer F.Cu) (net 6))
 (segment (start 65.024 77.597) (end 65.024 75.946) (width 0.254) (layer F.Cu) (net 4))
 (segment (start 65.659 75.311) (end 69.977 75.311) (width 0.254) (layer F.Cu) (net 4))
 (segment (start 65.024 75.946) (end 65.659 75.311) (width 0.254) (layer F.Cu) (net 4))
 (segment (start 72.898 79.121) (end 72.898 76.962) (width 0.254) (layer F.Cu) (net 3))
 (segment (start 72.009 76.073) (end 72.009 74.676) (width 0.254) (layer F.Cu) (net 3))
 (segment (start 72.898 76.962) (end 72.009 76.073) (width 0.254) (layer F.Cu) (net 3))
 (segment (start 76.327 75.311) (end 72.644 75.311) (width 0.254) (layer F.Cu) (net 3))
 (segment (start 72.009 74.676) (end 72.009 73.406) (width 0.254) (layer F.Cu) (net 3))
 (segment (start 72.644 75.311) (end 72.009 74.676) (width 0.254) (layer F.Cu) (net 3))
 (segment (start 72.009 68.199) (end 72.009 73.406) (width 0.254) (layer F.Cu) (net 3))
 (segment (start 71.374 74.041) (end 69.977 74.041) (width 0.254) (layer F.Cu) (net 3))
 (segment (start 72.009 73.406) (end 71.374 74.041) (width 0.254) (layer F.Cu) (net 3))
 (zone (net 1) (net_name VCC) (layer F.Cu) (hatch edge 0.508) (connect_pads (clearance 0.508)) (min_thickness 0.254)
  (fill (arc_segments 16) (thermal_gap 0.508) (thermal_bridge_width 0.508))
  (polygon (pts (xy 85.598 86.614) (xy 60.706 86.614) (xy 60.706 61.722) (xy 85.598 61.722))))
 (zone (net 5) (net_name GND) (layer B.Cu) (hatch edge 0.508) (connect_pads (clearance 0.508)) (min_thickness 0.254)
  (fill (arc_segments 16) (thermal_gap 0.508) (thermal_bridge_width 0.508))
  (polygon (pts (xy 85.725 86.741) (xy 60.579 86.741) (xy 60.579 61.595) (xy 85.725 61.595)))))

